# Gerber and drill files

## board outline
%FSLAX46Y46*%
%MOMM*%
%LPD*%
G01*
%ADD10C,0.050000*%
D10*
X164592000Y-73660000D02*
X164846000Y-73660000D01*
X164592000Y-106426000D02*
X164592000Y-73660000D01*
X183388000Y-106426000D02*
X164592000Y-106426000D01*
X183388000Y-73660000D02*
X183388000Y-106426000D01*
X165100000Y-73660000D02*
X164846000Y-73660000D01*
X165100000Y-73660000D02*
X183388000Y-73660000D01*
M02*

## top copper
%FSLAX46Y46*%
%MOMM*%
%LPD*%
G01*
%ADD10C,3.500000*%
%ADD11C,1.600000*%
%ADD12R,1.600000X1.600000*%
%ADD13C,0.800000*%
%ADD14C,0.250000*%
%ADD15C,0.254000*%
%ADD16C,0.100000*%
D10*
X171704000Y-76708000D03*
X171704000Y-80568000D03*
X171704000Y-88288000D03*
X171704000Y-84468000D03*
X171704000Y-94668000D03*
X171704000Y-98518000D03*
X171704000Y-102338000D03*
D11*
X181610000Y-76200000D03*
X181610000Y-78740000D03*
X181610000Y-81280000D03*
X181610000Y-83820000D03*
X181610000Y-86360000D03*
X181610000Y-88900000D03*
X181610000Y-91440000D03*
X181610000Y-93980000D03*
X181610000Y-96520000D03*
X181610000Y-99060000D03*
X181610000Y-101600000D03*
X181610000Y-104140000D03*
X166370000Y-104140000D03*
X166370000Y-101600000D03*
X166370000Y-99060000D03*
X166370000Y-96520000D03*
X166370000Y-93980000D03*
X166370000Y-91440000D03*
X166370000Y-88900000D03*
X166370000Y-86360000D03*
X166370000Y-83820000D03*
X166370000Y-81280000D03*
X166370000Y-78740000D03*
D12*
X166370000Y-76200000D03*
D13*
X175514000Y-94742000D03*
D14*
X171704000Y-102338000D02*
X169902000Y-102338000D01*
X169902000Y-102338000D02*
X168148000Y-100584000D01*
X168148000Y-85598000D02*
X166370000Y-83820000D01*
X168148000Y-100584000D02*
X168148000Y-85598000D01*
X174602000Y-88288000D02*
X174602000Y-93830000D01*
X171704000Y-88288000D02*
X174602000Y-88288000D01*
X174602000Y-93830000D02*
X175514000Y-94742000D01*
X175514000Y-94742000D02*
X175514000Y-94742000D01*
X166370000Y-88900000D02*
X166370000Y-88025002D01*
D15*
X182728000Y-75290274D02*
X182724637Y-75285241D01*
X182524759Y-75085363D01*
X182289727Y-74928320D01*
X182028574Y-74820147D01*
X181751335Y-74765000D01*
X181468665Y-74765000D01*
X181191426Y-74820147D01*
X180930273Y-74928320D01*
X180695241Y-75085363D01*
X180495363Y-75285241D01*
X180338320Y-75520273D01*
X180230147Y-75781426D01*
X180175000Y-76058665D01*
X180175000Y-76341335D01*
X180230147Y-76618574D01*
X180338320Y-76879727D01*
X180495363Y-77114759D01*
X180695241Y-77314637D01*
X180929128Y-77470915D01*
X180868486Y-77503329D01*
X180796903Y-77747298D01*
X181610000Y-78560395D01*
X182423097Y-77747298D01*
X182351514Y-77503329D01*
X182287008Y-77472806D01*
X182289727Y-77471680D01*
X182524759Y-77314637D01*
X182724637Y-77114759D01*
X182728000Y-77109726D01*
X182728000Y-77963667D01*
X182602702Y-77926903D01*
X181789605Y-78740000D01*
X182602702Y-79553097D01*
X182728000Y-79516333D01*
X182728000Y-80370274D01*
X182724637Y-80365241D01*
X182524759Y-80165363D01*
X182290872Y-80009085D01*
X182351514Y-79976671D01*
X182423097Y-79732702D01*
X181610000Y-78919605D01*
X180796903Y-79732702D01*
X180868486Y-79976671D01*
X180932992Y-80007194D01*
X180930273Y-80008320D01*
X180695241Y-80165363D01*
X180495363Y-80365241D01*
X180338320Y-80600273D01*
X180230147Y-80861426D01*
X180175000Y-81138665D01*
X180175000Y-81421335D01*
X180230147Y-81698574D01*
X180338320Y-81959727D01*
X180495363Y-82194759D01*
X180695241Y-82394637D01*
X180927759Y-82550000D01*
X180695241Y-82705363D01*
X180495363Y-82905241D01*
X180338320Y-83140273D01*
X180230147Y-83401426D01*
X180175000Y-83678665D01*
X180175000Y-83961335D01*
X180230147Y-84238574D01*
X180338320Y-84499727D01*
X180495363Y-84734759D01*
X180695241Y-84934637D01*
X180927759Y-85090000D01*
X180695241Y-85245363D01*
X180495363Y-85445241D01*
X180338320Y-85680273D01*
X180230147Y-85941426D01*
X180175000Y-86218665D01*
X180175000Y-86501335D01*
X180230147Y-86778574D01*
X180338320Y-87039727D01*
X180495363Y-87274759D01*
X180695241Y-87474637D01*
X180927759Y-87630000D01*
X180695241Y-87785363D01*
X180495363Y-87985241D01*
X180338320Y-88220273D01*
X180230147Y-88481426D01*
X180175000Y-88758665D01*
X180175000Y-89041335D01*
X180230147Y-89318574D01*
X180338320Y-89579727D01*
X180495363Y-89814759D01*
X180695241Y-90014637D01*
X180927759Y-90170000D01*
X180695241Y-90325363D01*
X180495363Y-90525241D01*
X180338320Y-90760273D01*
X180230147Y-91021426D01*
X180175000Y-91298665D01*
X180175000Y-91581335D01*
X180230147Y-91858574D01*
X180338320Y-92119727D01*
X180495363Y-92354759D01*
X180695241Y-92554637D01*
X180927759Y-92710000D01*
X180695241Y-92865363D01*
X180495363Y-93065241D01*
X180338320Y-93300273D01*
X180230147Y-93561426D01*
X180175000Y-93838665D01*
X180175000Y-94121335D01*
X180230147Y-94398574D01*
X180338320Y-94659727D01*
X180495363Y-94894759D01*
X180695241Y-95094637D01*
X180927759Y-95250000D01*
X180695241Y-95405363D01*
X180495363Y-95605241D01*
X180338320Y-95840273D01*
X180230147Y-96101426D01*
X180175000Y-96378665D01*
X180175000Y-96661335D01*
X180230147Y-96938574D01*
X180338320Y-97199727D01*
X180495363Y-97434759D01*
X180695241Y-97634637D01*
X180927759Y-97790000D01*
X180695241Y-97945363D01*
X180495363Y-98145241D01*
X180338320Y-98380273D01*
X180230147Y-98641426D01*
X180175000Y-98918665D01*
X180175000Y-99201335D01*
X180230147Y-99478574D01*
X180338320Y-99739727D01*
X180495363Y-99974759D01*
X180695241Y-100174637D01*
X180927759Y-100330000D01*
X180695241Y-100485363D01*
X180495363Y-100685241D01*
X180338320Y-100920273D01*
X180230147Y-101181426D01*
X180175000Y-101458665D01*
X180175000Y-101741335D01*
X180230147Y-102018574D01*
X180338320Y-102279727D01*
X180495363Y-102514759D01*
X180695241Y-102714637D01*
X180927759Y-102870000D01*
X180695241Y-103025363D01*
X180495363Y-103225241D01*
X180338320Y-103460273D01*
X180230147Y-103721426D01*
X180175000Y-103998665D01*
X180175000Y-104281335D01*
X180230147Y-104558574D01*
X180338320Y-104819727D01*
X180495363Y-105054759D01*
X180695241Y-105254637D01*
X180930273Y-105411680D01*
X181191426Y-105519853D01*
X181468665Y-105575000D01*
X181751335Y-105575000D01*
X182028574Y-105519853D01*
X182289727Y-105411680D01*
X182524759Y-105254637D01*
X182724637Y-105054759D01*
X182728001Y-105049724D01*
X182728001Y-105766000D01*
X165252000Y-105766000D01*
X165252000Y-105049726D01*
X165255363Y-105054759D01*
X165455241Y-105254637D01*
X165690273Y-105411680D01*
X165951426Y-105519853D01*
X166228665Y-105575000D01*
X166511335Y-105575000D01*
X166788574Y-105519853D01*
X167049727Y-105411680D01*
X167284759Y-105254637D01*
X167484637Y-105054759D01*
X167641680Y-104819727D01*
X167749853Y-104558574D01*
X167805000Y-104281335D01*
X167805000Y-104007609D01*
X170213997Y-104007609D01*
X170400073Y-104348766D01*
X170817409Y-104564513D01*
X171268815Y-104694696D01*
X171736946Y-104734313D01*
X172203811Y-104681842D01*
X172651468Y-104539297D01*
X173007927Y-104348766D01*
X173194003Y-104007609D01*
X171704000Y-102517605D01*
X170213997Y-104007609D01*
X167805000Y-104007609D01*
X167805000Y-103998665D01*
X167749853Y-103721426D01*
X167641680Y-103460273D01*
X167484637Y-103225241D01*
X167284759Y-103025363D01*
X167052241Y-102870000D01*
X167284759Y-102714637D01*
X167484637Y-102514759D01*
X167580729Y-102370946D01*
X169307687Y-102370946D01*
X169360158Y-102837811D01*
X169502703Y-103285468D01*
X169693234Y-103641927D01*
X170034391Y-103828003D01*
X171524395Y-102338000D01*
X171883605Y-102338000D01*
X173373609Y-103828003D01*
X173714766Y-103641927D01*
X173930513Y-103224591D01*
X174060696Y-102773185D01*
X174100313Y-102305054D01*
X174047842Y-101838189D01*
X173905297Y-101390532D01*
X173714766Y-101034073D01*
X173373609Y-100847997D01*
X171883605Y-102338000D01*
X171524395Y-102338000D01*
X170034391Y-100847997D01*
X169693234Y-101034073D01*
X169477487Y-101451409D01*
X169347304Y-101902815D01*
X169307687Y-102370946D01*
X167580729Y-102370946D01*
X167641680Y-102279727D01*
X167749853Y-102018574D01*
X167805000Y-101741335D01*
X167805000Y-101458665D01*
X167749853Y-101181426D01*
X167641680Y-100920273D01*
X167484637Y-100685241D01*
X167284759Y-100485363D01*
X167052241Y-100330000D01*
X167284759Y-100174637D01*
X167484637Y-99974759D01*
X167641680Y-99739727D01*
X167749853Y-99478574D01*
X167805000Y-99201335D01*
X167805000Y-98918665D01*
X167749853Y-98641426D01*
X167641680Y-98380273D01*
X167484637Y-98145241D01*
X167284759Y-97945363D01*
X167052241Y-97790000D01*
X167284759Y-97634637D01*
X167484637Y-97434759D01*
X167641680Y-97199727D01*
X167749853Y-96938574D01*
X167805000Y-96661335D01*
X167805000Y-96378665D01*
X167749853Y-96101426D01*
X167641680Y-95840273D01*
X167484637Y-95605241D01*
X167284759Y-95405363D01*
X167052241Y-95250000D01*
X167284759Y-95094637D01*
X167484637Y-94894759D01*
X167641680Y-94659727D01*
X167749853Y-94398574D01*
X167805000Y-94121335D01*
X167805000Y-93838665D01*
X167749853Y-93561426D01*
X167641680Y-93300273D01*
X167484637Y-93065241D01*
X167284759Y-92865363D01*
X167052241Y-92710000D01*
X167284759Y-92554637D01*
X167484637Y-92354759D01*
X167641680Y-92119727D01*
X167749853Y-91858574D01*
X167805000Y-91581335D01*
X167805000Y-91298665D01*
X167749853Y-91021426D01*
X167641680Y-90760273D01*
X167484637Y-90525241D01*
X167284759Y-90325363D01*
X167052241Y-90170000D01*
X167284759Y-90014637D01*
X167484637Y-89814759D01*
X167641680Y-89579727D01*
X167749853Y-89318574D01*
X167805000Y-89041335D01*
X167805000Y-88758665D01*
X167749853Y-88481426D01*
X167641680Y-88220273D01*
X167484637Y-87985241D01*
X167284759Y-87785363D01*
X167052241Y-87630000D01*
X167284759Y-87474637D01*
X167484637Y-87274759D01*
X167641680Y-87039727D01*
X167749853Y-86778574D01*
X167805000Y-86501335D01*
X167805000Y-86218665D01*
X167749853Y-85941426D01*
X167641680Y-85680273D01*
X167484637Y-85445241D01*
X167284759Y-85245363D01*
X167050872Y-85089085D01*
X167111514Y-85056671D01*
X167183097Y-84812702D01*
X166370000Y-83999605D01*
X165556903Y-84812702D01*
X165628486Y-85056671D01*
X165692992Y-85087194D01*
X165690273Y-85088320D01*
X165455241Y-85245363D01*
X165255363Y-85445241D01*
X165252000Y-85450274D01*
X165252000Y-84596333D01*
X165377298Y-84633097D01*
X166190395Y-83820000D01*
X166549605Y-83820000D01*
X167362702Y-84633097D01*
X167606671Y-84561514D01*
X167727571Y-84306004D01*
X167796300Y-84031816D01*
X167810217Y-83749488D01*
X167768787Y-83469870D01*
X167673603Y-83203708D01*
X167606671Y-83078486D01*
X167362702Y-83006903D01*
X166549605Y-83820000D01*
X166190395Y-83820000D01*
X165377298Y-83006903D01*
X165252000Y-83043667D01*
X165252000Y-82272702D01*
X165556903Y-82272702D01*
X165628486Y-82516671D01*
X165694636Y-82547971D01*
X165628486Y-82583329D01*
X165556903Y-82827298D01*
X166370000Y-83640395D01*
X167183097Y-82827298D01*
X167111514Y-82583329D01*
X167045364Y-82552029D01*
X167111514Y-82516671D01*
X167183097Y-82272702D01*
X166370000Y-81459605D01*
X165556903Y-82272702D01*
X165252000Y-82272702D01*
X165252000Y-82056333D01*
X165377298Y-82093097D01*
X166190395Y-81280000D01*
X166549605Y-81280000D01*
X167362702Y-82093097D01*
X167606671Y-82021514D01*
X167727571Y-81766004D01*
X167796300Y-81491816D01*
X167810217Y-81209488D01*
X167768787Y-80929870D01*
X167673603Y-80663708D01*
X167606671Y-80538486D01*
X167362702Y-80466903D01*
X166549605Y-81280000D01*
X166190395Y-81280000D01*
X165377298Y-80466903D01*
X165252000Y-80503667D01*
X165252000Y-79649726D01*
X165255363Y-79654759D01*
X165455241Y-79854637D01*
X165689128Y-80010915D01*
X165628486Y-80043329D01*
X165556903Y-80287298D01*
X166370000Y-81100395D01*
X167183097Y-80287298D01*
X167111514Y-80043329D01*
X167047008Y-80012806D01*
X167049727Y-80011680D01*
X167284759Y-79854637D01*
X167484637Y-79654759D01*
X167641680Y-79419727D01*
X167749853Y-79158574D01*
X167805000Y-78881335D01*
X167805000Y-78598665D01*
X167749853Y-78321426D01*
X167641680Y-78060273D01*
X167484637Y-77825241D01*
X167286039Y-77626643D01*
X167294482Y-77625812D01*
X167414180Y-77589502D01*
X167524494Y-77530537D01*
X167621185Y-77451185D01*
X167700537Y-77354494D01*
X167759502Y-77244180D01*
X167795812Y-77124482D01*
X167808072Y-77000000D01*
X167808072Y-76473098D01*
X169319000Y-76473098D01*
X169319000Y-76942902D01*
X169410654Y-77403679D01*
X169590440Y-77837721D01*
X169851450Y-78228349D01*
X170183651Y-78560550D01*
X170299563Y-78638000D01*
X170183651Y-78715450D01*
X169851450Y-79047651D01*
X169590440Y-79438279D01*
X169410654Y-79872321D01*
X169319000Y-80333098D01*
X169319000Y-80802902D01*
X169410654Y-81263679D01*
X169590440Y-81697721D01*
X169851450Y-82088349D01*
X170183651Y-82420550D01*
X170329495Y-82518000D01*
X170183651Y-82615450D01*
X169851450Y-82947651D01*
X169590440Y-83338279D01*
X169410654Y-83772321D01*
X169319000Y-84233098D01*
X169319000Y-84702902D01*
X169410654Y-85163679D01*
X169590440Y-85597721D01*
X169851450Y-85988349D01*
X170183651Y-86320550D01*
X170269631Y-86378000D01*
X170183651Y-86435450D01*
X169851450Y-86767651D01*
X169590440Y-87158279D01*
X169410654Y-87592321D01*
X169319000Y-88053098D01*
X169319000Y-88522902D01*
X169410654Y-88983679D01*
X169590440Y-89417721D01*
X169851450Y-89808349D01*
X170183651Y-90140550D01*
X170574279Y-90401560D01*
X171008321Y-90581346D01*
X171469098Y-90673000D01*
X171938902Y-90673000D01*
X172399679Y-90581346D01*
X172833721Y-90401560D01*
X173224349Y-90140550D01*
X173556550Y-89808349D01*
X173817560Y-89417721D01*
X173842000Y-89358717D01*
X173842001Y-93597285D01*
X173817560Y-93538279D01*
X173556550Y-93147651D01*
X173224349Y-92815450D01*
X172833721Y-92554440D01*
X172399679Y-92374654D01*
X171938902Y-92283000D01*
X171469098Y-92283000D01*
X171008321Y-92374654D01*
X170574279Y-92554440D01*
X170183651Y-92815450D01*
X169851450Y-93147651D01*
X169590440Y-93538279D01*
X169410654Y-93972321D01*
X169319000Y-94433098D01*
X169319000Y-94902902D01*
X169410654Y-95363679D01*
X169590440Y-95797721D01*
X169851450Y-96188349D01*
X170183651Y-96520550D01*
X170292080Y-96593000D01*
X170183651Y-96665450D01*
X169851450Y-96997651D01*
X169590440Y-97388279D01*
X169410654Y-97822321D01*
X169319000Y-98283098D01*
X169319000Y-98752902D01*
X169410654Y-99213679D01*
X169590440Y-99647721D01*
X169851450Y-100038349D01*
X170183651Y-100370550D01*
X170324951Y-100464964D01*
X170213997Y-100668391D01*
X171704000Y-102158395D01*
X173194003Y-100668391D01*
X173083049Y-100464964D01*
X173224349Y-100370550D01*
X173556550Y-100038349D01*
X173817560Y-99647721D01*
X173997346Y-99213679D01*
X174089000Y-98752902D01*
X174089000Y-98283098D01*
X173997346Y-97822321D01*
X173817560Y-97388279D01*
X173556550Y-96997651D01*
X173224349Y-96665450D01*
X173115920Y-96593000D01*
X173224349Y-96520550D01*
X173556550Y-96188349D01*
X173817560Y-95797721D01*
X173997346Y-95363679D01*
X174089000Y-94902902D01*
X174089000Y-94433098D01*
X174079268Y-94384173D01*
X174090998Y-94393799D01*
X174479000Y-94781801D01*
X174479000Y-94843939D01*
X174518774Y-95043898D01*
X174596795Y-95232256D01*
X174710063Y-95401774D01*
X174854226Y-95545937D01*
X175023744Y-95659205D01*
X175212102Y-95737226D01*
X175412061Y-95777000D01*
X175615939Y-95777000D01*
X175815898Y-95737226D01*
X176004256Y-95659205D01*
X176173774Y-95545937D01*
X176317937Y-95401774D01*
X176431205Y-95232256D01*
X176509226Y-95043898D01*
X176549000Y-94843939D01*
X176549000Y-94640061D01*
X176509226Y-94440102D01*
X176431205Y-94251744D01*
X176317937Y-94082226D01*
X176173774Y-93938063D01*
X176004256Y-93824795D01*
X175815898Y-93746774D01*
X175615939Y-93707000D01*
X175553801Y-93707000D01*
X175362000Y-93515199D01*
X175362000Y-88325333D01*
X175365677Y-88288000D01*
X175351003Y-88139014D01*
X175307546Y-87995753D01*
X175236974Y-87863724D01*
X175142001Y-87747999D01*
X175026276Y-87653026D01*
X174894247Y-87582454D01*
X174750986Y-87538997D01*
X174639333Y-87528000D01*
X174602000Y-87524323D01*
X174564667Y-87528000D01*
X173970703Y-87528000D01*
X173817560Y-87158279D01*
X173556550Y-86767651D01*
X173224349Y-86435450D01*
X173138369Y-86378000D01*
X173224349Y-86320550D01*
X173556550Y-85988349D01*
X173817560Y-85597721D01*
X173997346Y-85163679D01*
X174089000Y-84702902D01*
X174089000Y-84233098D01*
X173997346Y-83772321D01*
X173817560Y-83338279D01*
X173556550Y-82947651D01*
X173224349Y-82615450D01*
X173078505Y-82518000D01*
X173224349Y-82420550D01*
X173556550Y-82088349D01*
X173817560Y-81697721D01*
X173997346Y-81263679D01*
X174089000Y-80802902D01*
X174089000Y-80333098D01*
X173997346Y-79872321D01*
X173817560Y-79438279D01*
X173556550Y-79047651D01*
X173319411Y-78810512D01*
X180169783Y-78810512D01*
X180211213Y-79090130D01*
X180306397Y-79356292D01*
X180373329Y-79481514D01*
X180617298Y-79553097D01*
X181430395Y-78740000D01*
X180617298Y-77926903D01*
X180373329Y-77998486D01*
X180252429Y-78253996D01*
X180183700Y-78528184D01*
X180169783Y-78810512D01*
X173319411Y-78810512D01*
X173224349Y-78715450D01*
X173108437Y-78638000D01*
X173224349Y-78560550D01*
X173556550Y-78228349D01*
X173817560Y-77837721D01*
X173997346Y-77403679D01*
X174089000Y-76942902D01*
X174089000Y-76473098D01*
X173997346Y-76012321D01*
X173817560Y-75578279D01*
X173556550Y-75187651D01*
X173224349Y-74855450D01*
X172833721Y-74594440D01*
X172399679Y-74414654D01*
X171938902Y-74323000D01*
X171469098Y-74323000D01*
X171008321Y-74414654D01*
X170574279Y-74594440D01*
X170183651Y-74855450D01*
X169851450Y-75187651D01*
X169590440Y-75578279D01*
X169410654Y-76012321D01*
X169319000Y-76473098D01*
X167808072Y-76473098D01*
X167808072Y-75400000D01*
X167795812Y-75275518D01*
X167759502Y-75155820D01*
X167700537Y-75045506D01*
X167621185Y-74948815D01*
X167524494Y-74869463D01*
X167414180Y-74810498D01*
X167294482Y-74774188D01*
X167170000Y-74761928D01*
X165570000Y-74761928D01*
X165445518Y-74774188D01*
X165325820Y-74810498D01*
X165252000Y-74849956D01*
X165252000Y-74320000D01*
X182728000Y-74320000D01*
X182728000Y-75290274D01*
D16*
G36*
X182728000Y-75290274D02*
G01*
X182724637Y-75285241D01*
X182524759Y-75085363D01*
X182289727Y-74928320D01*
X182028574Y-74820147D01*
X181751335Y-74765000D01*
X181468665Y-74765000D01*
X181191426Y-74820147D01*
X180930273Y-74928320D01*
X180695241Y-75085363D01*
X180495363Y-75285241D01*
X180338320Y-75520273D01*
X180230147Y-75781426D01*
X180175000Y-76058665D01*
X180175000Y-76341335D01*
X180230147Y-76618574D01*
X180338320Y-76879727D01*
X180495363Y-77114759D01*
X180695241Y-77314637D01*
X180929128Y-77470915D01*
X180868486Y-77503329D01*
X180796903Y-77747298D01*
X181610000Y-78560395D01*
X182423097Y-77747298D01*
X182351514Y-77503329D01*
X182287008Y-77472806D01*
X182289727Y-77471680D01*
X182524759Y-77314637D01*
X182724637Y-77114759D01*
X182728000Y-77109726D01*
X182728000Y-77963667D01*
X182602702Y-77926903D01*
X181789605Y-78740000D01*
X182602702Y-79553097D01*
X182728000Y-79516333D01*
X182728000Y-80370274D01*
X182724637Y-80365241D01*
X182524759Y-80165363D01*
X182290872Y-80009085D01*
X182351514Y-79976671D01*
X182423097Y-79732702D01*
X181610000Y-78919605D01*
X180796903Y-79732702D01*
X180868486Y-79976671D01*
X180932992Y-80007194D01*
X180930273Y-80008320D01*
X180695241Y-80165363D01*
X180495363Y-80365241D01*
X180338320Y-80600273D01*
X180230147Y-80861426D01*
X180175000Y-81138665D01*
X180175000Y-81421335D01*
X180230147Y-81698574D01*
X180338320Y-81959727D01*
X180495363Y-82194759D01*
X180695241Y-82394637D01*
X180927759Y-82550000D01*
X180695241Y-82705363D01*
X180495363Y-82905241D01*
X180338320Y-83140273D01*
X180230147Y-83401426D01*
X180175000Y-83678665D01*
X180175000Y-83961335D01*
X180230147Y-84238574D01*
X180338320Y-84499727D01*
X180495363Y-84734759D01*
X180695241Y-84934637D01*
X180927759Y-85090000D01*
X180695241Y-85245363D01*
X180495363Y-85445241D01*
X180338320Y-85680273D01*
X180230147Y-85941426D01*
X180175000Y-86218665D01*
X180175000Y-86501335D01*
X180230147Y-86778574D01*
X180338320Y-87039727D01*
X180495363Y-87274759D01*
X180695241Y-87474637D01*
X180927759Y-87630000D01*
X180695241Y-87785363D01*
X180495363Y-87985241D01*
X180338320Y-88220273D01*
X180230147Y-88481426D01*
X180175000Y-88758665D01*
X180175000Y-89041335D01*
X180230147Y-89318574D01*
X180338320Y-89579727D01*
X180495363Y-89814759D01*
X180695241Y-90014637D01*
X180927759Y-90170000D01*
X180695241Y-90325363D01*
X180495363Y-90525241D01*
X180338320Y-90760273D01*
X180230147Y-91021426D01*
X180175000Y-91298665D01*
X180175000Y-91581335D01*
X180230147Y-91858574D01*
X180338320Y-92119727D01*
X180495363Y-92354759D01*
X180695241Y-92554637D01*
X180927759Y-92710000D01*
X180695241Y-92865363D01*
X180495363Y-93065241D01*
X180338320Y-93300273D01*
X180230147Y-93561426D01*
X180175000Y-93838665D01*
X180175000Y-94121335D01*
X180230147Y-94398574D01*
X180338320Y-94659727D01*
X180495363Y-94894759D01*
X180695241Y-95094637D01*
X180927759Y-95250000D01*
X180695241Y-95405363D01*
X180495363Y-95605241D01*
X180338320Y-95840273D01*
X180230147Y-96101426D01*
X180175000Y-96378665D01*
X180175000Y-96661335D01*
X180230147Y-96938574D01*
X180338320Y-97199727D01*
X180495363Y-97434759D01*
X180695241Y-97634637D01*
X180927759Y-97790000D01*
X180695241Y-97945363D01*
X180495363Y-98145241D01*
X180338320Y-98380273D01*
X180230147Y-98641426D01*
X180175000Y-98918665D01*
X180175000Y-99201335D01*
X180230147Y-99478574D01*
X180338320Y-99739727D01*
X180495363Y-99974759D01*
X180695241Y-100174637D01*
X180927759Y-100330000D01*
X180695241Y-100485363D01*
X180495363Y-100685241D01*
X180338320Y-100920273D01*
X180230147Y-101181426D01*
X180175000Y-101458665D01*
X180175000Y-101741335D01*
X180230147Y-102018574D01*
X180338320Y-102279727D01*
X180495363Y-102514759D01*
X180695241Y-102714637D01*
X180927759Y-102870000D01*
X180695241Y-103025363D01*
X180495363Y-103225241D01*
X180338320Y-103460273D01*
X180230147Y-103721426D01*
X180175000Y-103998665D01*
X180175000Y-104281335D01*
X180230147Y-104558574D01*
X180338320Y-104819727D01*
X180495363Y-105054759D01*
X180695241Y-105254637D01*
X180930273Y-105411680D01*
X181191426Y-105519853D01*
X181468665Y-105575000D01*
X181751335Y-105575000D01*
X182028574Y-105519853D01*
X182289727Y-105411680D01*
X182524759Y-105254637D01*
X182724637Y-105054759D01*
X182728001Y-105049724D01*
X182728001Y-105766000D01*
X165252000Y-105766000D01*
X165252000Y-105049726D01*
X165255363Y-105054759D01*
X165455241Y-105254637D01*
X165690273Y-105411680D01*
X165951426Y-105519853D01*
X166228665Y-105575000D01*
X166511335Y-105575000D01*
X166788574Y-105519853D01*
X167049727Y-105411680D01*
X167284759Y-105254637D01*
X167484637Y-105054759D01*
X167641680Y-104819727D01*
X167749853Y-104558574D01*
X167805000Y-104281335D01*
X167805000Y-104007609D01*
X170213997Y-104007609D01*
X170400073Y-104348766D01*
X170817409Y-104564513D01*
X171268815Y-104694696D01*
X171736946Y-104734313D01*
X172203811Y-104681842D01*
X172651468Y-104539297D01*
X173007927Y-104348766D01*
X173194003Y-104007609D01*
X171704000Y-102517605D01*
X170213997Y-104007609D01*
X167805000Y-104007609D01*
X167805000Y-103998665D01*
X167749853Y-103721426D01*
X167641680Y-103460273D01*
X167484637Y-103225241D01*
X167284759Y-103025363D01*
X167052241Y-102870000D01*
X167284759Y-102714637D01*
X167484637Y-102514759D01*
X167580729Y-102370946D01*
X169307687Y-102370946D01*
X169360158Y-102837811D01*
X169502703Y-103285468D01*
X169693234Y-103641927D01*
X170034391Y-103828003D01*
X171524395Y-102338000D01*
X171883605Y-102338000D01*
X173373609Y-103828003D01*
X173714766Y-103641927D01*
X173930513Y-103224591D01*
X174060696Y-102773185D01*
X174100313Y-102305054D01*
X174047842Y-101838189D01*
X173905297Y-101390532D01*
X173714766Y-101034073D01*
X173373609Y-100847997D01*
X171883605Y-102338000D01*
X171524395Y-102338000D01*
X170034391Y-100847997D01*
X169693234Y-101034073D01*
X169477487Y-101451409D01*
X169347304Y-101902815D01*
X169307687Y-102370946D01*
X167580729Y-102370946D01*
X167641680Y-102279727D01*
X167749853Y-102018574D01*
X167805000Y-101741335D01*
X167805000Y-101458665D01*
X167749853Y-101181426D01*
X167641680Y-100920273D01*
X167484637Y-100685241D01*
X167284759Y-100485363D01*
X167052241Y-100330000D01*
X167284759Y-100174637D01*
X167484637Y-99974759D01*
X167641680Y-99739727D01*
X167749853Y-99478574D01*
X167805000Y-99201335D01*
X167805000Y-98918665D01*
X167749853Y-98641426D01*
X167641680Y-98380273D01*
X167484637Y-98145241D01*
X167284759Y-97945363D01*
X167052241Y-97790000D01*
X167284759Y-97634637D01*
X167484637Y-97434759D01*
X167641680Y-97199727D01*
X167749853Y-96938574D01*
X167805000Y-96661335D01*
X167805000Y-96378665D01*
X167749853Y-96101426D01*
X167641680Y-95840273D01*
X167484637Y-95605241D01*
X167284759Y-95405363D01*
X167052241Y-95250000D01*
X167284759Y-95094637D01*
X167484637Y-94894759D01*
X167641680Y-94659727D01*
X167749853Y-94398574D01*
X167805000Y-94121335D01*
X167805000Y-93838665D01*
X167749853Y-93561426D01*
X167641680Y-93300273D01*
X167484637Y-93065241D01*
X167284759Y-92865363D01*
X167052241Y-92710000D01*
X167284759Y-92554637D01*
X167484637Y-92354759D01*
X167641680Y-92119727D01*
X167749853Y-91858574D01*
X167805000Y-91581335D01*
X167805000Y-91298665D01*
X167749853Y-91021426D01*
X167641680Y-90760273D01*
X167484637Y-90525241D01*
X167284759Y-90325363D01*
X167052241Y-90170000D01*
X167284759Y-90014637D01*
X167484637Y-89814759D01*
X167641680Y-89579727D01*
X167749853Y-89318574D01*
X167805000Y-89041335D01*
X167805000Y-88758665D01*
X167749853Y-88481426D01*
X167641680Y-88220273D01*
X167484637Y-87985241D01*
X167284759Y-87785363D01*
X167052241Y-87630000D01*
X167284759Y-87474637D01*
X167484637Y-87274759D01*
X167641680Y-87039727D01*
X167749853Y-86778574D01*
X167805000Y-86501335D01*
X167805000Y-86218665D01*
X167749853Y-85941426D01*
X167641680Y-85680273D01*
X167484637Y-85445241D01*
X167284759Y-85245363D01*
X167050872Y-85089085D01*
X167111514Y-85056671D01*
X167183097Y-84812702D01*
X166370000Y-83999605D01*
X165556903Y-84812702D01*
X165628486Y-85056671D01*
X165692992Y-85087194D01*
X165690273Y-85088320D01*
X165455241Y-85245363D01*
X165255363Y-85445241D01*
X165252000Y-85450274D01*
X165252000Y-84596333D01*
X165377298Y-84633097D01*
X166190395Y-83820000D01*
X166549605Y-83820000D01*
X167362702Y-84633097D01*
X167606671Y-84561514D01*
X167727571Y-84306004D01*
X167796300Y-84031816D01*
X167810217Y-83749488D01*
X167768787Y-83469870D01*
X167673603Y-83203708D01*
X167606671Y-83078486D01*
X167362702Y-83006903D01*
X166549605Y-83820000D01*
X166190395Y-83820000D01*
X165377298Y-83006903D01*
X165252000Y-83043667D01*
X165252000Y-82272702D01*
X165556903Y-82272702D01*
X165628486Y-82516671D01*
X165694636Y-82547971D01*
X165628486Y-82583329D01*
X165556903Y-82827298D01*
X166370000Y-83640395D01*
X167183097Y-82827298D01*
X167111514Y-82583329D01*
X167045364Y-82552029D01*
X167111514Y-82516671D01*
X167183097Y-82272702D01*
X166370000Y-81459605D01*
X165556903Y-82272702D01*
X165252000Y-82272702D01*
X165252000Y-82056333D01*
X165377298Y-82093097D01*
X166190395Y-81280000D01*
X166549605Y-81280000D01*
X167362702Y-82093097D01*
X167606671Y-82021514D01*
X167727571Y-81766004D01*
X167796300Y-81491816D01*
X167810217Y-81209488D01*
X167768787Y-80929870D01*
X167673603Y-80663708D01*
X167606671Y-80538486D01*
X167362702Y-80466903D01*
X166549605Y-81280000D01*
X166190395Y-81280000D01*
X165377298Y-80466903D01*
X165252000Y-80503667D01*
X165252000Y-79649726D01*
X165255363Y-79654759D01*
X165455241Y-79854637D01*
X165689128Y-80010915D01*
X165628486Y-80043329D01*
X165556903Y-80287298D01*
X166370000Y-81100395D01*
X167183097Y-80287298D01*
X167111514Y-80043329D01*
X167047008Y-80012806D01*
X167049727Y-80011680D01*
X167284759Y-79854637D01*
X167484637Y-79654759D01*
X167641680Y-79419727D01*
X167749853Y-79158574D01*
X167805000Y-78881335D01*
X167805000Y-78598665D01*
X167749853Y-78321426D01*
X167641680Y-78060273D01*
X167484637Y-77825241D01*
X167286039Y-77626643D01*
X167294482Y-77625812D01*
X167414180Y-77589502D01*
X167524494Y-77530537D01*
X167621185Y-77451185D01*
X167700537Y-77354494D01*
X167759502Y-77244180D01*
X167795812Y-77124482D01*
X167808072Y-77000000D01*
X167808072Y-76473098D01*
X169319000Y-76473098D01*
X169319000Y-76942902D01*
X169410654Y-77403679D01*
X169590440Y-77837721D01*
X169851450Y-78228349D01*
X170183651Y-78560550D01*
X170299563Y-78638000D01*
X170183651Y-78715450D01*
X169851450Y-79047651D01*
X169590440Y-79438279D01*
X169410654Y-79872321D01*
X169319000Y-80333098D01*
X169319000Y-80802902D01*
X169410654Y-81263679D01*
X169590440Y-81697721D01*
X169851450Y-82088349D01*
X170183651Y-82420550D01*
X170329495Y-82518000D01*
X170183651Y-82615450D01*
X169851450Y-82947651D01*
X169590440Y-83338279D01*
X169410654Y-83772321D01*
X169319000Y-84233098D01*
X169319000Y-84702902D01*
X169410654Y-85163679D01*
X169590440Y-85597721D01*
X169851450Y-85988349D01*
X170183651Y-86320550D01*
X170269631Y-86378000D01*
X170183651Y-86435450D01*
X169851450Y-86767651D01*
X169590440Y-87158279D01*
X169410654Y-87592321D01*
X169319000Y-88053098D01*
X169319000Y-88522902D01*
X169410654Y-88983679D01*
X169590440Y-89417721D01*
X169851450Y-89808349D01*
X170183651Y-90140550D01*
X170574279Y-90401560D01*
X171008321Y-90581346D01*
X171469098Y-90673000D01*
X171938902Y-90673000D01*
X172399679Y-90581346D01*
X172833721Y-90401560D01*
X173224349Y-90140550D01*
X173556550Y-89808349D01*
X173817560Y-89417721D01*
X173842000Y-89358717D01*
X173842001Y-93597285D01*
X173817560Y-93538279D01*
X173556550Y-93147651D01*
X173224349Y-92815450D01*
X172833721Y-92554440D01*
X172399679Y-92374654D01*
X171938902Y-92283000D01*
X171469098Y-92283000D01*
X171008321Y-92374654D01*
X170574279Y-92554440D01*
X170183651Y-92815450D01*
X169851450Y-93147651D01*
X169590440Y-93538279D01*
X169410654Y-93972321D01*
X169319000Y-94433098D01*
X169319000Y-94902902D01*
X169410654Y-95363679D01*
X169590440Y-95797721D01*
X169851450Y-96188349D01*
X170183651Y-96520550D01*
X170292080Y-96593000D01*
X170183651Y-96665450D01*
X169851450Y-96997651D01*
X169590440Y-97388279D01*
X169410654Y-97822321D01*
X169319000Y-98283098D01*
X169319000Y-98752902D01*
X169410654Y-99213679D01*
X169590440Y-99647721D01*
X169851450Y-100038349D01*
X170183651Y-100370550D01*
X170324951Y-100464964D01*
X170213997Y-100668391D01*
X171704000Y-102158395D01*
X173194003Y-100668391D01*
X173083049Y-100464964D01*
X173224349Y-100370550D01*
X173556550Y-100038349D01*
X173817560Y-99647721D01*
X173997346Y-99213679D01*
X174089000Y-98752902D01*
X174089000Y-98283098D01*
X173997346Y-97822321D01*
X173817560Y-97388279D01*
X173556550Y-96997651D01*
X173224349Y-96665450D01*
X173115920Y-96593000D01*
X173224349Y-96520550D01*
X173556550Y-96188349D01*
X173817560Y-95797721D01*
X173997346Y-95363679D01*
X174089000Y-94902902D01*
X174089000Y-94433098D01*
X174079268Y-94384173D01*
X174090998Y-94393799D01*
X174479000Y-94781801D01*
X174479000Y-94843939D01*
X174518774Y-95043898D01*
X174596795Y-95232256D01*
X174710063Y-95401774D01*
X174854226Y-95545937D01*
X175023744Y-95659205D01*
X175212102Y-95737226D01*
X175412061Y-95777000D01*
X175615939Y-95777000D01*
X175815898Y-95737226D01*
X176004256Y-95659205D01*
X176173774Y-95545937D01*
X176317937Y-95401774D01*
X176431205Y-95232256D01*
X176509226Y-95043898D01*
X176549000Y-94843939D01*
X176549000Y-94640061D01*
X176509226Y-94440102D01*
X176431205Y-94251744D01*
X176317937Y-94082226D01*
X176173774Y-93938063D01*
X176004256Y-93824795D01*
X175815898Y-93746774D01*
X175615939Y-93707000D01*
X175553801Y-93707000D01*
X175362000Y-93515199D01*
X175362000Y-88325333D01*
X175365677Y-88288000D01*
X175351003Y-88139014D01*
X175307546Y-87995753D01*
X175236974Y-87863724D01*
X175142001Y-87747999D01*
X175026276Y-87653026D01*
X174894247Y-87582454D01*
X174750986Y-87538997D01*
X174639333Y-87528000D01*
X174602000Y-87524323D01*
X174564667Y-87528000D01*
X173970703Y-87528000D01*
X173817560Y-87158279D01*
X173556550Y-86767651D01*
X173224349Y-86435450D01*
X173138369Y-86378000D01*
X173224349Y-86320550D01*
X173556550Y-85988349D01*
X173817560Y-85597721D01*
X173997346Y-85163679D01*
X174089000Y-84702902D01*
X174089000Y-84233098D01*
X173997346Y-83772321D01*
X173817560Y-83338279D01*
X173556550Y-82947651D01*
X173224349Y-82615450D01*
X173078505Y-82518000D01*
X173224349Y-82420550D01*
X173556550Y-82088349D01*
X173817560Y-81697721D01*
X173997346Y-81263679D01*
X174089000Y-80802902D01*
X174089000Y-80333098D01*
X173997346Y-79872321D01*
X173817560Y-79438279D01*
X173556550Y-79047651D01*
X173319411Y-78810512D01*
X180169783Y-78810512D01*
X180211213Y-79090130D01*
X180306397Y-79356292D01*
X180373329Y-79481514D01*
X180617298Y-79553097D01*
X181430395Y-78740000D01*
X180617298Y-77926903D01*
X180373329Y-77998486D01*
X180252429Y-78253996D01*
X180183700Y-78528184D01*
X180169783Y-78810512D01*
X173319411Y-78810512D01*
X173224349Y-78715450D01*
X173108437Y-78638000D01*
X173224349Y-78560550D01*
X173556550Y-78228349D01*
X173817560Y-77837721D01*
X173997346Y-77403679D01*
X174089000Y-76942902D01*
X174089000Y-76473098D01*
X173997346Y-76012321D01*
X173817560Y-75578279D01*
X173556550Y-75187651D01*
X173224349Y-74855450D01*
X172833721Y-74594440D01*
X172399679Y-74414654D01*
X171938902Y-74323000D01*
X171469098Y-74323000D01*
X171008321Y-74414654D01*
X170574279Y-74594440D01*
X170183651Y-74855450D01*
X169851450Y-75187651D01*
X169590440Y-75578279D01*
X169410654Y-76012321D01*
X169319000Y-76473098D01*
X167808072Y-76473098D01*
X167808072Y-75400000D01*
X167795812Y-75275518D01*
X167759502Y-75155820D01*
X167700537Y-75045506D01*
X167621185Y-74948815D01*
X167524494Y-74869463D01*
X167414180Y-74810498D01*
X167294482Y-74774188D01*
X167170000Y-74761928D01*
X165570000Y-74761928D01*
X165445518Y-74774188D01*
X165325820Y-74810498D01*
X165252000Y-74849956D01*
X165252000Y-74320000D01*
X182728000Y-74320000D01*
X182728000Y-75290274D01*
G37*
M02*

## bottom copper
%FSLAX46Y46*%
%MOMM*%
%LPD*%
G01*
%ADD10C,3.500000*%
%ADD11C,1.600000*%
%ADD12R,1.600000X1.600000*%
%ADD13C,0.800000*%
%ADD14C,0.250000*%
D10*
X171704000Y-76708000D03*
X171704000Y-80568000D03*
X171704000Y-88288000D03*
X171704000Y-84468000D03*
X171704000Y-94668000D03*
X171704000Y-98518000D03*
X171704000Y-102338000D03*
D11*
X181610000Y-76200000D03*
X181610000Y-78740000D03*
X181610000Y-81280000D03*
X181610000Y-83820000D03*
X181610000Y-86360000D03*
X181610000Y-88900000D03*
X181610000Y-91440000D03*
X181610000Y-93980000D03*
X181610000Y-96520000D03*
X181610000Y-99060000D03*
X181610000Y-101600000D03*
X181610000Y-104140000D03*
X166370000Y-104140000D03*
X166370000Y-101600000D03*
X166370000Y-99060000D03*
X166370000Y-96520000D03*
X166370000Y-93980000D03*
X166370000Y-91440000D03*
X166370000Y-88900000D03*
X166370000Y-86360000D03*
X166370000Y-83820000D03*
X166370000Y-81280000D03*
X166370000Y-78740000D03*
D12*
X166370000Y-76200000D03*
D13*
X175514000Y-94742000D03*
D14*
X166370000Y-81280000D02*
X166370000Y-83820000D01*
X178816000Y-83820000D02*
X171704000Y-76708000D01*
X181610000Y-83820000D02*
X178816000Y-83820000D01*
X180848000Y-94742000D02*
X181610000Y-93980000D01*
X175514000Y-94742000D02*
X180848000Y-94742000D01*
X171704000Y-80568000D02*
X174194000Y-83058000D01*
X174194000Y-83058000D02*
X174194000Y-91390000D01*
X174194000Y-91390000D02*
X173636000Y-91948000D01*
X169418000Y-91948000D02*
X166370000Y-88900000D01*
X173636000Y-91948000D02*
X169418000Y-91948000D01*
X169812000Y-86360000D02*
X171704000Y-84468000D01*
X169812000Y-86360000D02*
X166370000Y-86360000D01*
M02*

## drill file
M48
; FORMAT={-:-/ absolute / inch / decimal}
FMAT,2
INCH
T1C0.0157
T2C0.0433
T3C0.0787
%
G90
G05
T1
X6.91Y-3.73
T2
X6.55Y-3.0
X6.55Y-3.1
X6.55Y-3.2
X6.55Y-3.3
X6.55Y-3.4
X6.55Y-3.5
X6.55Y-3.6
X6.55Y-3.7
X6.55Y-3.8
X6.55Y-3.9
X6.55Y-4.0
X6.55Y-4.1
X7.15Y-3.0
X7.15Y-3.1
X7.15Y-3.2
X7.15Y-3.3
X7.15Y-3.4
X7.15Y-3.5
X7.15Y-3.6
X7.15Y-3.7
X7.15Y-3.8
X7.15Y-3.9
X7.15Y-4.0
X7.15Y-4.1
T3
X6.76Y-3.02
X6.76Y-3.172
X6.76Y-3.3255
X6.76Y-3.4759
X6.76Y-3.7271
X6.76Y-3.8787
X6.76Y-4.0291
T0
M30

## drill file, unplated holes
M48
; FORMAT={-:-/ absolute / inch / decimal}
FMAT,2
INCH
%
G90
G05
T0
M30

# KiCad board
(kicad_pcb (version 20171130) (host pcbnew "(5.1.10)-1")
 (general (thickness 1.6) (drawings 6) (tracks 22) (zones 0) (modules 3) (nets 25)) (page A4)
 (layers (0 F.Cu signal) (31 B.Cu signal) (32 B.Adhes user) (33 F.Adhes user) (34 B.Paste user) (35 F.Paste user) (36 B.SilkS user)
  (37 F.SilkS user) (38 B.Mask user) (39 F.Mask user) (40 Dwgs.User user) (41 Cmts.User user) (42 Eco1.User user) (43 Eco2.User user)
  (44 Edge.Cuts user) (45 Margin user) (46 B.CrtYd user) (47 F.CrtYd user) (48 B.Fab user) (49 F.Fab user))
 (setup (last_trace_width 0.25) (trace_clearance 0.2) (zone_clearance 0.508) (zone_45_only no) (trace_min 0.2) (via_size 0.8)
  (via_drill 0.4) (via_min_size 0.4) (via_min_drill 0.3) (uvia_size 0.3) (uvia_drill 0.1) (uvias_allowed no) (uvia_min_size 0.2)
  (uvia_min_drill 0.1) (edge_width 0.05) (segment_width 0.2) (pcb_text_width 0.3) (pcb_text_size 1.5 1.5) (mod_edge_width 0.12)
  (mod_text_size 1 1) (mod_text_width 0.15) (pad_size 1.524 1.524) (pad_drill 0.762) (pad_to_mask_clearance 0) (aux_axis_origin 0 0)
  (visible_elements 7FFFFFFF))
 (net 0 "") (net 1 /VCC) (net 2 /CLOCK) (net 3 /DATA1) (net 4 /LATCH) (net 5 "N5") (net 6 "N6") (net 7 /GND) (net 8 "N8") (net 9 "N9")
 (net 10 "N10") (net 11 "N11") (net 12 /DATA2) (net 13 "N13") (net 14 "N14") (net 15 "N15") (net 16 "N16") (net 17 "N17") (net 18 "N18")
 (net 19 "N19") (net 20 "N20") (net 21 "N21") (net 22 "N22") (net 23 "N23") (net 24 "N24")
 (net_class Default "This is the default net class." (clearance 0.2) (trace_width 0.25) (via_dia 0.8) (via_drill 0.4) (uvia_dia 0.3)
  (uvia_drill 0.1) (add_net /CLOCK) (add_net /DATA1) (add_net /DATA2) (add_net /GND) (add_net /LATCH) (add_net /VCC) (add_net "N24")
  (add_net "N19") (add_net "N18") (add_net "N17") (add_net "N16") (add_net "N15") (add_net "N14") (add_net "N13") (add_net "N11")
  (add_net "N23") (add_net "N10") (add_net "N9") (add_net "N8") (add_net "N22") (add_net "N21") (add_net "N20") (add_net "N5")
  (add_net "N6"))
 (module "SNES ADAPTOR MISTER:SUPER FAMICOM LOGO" (layer F.Cu) (at 178.054 89.154 270)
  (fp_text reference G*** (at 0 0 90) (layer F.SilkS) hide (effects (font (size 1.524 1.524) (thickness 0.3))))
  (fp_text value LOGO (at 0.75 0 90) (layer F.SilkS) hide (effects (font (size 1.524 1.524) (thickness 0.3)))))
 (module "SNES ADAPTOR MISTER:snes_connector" (layer F.Cu) (at 171.704 86.868 270)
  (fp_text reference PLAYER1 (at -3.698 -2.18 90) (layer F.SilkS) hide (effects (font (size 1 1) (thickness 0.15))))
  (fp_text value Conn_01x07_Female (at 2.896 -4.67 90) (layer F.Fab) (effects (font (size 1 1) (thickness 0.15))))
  (pad 1 thru_hole circle (at -10.16 0 270) (size 3.5 3.5) (drill 2) (layers *.Cu *.Mask) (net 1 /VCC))
  (pad 2 thru_hole circle (at -6.3 0 270) (size 3.5 3.5) (drill 2) (layers *.Cu *.Mask) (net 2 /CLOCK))
  (pad 4 thru_hole circle (at 1.42 0 270) (size 3.5 3.5) (drill 2) (layers *.Cu *.Mask) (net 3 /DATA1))
  (pad 3 thru_hole circle (at -2.4 0 270) (size 3.5 3.5) (drill 2) (layers *.Cu *.Mask) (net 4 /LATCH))
  (pad 5 thru_hole circle (at 7.8 0 270) (size 3.5 3.5) (drill 2) (layers *.Cu *.Mask) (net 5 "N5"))
  (pad 6 thru_hole circle (at 11.65 0 270) (size 3.5 3.5) (drill 2) (layers *.Cu *.Mask) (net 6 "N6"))
  (pad 7 thru_hole circle (at 15.47 0 270) (size 3.5 3.5) (drill 2) (layers *.Cu *.Mask) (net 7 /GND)))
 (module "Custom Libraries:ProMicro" (layer F.Cu) (at 173.99 90.17 270)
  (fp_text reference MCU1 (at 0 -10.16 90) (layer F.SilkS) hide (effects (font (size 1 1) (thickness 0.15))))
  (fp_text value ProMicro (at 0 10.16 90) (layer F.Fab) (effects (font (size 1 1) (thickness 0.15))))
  (pad 24 thru_hole circle (at -13.97 -7.62 270) (size 1.6 1.6) (drill 1.1) (layers *.Cu *.Mask F.SilkS) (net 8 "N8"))
  (pad 23 thru_hole circle (at -11.43 -7.62 270) (size 1.6 1.6) (drill 1.1) (layers *.Cu *.Mask F.SilkS) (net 7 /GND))
  (pad 22 thru_hole circle (at -8.89 -7.62 270) (size 1.6 1.6) (drill 1.1) (layers *.Cu *.Mask F.SilkS) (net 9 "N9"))
  (pad 21 thru_hole circle (at -6.35 -7.62 270) (size 1.6 1.6) (drill 1.1) (layers *.Cu *.Mask F.SilkS) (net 1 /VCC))
  (pad 20 thru_hole circle (at -3.81 -7.62 270) (size 1.6 1.6) (drill 1.1) (layers *.Cu *.Mask F.SilkS) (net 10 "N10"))
  (pad 19 thru_hole circle (at -1.27 -7.62 270) (size 1.6 1.6) (drill 1.1) (layers *.Cu *.Mask F.SilkS) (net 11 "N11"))
  (pad 18 thru_hole circle (at 1.27 -7.62 270) (size 1.6 1.6) (drill 1.1) (layers *.Cu *.Mask F.SilkS) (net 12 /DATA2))
  (pad 17 thru_hole circle (at 3.81 -7.62 270) (size 1.6 1.6) (drill 1.1) (layers *.Cu *.Mask F.SilkS) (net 3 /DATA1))
  (pad 16 thru_hole circle (at 6.35 -7.62 270) (size 1.6 1.6) (drill 1.1) (layers *.Cu *.Mask F.SilkS) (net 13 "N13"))
  (pad 15 thru_hole circle (at 8.89 -7.62 270) (size 1.6 1.6) (drill 1.1) (layers *.Cu *.Mask F.SilkS) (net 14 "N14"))
  (pad 14 thru_hole circle (at 11.43 -7.62 270) (size 1.6 1.6) (drill 1.1) (layers *.Cu *.Mask F.SilkS) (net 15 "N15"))
  (pad 13 thru_hole circle (at 13.97 -7.62 270) (size 1.6 1.6) (drill 1.1) (layers *.Cu *.Mask F.SilkS) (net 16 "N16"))
  (pad 12 thru_hole circle (at 13.97 7.62 270) (size 1.6 1.6) (drill 1.1) (layers *.Cu *.Mask F.SilkS) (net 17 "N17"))
  (pad 11 thru_hole circle (at 11.43 7.62 270) (size 1.6 1.6) (drill 1.1) (layers *.Cu *.Mask F.SilkS) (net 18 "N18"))
  (pad 10 thru_hole circle (at 8.89 7.62 270) (size 1.6 1.6) (drill 1.1) (layers *.Cu *.Mask F.SilkS) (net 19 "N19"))
  (pad 9 thru_hole circle (at 6.35 7.62 270) (size 1.6 1.6) (drill 1.1) (layers *.Cu *.Mask F.SilkS) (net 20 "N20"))
  (pad 8 thru_hole circle (at 3.81 7.62 270) (size 1.6 1.6) (drill 1.1) (layers *.Cu *.Mask F.SilkS) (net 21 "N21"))
  (pad 7 thru_hole circle (at 1.27 7.62 270) (size 1.6 1.6) (drill 1.1) (layers *.Cu *.Mask F.SilkS) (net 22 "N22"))
  (pad 6 thru_hole circle (at -1.27 7.62 270) (size 1.6 1.6) (drill 1.1) (layers *.Cu *.Mask F.SilkS) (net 2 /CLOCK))
  (pad 5 thru_hole circle (at -3.81 7.62 270) (size 1.6 1.6) (drill 1.1) (layers *.Cu *.Mask F.SilkS) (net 4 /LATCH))
  (pad 4 thru_hole circle (at -6.35 7.62 270) (size 1.6 1.6) (drill 1.1) (layers *.Cu *.Mask F.SilkS) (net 7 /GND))
  (pad 3 thru_hole circle (at -8.89 7.62 270) (size 1.6 1.6) (drill 1.1) (layers *.Cu *.Mask F.SilkS) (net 7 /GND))
  (pad 2 thru_hole circle (at -11.43 7.62 270) (size 1.6 1.6) (drill 1.1) (layers *.Cu *.Mask F.SilkS) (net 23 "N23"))
  (pad 1 thru_hole rect (at -13.97 7.62 270) (size 1.6 1.6) (drill 1.1) (layers *.Cu *.Mask F.SilkS) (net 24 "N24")))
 (gr_line (start 164.592 73.66) (end 164.846 73.66) (layer Edge.Cuts) (width 0.05))
 (gr_line (start 164.592 106.426) (end 164.592 73.66) (layer Edge.Cuts) (width 0.05))
 (gr_line (start 183.388 106.426) (end 164.592 106.426) (layer Edge.Cuts) (width 0.05))
 (gr_line (start 183.388 73.66) (end 183.388 106.426) (layer Edge.Cuts) (width 0.05))
 (gr_line (start 165.1 73.66) (end 164.846 73.66) (layer Edge.Cuts) (width 0.05))
 (gr_line (start 165.1 73.66) (end 183.388 73.66) (layer Edge.Cuts) (width 0.05))
 (segment (start 166.37 81.28) (end 166.37 83.82) (width 0.25) (layer B.Cu) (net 7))
 (segment (start 171.704 102.338) (end 169.902 102.338) (width 0.25) (layer F.Cu) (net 7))
 (segment (start 169.902 102.338) (end 168.148 100.584) (width 0.25) (layer F.Cu) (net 7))
 (segment (start 168.148 85.598) (end 166.37 83.82) (width 0.25) (layer F.Cu) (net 7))
 (segment (start 168.148 100.584) (end 168.148 85.598) (width 0.25) (layer F.Cu) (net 7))
 (segment (start 178.816 83.82) (end 171.704 76.708) (width 0.25) (layer B.Cu) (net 1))
 (segment (start 181.61 83.82) (end 178.816 83.82) (width 0.25) (layer B.Cu) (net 1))
 (segment (start 174.602 88.288) (end 174.602 93.83) (width 0.25) (layer F.Cu) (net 3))
 (segment (start 171.704 88.288) (end 174.602 88.288) (width 0.25) (layer F.Cu) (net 3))
 (segment (start 174.602 93.83) (end 175.514 94.742) (width 0.25) (layer F.Cu) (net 3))
 (segment (start 175.514 94.742) (end 175.514 94.742) (width 0.25) (layer F.Cu) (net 3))
 (via (at 175.514 94.742) (size 0.8) (drill 0.4) (layers F.Cu B.Cu) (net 3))
 (segment (start 180.848 94.742) (end 181.61 93.98) (width 0.25) (layer B.Cu) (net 3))
 (segment (start 175.514 94.742) (end 180.848 94.742) (width 0.25) (layer B.Cu) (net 3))
 (segment (start 166.37 88.9) (end 166.37 88.025002) (width 0.25) (layer F.Cu) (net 2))
 (segment (start 171.704 80.568) (end 174.194 83.058) (width 0.25) (layer B.Cu) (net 2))
 (segment (start 174.194 83.058) (end 174.194 91.39) (width 0.25) (layer B.Cu) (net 2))
 (segment (start 174.194 91.39) (end 173.636 91.948) (width 0.25) (layer B.Cu) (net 2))
 (segment (start 169.418 91.948) (end 166.37 88.9) (width 0.25) (layer B.Cu) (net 2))
 (segment (start 173.636 91.948) (end 169.418 91.948) (width 0.25) (layer B.Cu) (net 2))
 (segment (start 169.812 86.36) (end 171.704 84.468) (width 0.25) (layer B.Cu) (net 4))
 (segment (start 169.812 86.36) (end 166.37 86.36) (width 0.25) (layer B.Cu) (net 4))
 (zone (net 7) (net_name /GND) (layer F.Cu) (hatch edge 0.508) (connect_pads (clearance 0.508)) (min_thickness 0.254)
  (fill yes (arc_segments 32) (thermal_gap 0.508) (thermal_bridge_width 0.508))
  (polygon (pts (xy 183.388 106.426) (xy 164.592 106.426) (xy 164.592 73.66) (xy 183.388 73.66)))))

